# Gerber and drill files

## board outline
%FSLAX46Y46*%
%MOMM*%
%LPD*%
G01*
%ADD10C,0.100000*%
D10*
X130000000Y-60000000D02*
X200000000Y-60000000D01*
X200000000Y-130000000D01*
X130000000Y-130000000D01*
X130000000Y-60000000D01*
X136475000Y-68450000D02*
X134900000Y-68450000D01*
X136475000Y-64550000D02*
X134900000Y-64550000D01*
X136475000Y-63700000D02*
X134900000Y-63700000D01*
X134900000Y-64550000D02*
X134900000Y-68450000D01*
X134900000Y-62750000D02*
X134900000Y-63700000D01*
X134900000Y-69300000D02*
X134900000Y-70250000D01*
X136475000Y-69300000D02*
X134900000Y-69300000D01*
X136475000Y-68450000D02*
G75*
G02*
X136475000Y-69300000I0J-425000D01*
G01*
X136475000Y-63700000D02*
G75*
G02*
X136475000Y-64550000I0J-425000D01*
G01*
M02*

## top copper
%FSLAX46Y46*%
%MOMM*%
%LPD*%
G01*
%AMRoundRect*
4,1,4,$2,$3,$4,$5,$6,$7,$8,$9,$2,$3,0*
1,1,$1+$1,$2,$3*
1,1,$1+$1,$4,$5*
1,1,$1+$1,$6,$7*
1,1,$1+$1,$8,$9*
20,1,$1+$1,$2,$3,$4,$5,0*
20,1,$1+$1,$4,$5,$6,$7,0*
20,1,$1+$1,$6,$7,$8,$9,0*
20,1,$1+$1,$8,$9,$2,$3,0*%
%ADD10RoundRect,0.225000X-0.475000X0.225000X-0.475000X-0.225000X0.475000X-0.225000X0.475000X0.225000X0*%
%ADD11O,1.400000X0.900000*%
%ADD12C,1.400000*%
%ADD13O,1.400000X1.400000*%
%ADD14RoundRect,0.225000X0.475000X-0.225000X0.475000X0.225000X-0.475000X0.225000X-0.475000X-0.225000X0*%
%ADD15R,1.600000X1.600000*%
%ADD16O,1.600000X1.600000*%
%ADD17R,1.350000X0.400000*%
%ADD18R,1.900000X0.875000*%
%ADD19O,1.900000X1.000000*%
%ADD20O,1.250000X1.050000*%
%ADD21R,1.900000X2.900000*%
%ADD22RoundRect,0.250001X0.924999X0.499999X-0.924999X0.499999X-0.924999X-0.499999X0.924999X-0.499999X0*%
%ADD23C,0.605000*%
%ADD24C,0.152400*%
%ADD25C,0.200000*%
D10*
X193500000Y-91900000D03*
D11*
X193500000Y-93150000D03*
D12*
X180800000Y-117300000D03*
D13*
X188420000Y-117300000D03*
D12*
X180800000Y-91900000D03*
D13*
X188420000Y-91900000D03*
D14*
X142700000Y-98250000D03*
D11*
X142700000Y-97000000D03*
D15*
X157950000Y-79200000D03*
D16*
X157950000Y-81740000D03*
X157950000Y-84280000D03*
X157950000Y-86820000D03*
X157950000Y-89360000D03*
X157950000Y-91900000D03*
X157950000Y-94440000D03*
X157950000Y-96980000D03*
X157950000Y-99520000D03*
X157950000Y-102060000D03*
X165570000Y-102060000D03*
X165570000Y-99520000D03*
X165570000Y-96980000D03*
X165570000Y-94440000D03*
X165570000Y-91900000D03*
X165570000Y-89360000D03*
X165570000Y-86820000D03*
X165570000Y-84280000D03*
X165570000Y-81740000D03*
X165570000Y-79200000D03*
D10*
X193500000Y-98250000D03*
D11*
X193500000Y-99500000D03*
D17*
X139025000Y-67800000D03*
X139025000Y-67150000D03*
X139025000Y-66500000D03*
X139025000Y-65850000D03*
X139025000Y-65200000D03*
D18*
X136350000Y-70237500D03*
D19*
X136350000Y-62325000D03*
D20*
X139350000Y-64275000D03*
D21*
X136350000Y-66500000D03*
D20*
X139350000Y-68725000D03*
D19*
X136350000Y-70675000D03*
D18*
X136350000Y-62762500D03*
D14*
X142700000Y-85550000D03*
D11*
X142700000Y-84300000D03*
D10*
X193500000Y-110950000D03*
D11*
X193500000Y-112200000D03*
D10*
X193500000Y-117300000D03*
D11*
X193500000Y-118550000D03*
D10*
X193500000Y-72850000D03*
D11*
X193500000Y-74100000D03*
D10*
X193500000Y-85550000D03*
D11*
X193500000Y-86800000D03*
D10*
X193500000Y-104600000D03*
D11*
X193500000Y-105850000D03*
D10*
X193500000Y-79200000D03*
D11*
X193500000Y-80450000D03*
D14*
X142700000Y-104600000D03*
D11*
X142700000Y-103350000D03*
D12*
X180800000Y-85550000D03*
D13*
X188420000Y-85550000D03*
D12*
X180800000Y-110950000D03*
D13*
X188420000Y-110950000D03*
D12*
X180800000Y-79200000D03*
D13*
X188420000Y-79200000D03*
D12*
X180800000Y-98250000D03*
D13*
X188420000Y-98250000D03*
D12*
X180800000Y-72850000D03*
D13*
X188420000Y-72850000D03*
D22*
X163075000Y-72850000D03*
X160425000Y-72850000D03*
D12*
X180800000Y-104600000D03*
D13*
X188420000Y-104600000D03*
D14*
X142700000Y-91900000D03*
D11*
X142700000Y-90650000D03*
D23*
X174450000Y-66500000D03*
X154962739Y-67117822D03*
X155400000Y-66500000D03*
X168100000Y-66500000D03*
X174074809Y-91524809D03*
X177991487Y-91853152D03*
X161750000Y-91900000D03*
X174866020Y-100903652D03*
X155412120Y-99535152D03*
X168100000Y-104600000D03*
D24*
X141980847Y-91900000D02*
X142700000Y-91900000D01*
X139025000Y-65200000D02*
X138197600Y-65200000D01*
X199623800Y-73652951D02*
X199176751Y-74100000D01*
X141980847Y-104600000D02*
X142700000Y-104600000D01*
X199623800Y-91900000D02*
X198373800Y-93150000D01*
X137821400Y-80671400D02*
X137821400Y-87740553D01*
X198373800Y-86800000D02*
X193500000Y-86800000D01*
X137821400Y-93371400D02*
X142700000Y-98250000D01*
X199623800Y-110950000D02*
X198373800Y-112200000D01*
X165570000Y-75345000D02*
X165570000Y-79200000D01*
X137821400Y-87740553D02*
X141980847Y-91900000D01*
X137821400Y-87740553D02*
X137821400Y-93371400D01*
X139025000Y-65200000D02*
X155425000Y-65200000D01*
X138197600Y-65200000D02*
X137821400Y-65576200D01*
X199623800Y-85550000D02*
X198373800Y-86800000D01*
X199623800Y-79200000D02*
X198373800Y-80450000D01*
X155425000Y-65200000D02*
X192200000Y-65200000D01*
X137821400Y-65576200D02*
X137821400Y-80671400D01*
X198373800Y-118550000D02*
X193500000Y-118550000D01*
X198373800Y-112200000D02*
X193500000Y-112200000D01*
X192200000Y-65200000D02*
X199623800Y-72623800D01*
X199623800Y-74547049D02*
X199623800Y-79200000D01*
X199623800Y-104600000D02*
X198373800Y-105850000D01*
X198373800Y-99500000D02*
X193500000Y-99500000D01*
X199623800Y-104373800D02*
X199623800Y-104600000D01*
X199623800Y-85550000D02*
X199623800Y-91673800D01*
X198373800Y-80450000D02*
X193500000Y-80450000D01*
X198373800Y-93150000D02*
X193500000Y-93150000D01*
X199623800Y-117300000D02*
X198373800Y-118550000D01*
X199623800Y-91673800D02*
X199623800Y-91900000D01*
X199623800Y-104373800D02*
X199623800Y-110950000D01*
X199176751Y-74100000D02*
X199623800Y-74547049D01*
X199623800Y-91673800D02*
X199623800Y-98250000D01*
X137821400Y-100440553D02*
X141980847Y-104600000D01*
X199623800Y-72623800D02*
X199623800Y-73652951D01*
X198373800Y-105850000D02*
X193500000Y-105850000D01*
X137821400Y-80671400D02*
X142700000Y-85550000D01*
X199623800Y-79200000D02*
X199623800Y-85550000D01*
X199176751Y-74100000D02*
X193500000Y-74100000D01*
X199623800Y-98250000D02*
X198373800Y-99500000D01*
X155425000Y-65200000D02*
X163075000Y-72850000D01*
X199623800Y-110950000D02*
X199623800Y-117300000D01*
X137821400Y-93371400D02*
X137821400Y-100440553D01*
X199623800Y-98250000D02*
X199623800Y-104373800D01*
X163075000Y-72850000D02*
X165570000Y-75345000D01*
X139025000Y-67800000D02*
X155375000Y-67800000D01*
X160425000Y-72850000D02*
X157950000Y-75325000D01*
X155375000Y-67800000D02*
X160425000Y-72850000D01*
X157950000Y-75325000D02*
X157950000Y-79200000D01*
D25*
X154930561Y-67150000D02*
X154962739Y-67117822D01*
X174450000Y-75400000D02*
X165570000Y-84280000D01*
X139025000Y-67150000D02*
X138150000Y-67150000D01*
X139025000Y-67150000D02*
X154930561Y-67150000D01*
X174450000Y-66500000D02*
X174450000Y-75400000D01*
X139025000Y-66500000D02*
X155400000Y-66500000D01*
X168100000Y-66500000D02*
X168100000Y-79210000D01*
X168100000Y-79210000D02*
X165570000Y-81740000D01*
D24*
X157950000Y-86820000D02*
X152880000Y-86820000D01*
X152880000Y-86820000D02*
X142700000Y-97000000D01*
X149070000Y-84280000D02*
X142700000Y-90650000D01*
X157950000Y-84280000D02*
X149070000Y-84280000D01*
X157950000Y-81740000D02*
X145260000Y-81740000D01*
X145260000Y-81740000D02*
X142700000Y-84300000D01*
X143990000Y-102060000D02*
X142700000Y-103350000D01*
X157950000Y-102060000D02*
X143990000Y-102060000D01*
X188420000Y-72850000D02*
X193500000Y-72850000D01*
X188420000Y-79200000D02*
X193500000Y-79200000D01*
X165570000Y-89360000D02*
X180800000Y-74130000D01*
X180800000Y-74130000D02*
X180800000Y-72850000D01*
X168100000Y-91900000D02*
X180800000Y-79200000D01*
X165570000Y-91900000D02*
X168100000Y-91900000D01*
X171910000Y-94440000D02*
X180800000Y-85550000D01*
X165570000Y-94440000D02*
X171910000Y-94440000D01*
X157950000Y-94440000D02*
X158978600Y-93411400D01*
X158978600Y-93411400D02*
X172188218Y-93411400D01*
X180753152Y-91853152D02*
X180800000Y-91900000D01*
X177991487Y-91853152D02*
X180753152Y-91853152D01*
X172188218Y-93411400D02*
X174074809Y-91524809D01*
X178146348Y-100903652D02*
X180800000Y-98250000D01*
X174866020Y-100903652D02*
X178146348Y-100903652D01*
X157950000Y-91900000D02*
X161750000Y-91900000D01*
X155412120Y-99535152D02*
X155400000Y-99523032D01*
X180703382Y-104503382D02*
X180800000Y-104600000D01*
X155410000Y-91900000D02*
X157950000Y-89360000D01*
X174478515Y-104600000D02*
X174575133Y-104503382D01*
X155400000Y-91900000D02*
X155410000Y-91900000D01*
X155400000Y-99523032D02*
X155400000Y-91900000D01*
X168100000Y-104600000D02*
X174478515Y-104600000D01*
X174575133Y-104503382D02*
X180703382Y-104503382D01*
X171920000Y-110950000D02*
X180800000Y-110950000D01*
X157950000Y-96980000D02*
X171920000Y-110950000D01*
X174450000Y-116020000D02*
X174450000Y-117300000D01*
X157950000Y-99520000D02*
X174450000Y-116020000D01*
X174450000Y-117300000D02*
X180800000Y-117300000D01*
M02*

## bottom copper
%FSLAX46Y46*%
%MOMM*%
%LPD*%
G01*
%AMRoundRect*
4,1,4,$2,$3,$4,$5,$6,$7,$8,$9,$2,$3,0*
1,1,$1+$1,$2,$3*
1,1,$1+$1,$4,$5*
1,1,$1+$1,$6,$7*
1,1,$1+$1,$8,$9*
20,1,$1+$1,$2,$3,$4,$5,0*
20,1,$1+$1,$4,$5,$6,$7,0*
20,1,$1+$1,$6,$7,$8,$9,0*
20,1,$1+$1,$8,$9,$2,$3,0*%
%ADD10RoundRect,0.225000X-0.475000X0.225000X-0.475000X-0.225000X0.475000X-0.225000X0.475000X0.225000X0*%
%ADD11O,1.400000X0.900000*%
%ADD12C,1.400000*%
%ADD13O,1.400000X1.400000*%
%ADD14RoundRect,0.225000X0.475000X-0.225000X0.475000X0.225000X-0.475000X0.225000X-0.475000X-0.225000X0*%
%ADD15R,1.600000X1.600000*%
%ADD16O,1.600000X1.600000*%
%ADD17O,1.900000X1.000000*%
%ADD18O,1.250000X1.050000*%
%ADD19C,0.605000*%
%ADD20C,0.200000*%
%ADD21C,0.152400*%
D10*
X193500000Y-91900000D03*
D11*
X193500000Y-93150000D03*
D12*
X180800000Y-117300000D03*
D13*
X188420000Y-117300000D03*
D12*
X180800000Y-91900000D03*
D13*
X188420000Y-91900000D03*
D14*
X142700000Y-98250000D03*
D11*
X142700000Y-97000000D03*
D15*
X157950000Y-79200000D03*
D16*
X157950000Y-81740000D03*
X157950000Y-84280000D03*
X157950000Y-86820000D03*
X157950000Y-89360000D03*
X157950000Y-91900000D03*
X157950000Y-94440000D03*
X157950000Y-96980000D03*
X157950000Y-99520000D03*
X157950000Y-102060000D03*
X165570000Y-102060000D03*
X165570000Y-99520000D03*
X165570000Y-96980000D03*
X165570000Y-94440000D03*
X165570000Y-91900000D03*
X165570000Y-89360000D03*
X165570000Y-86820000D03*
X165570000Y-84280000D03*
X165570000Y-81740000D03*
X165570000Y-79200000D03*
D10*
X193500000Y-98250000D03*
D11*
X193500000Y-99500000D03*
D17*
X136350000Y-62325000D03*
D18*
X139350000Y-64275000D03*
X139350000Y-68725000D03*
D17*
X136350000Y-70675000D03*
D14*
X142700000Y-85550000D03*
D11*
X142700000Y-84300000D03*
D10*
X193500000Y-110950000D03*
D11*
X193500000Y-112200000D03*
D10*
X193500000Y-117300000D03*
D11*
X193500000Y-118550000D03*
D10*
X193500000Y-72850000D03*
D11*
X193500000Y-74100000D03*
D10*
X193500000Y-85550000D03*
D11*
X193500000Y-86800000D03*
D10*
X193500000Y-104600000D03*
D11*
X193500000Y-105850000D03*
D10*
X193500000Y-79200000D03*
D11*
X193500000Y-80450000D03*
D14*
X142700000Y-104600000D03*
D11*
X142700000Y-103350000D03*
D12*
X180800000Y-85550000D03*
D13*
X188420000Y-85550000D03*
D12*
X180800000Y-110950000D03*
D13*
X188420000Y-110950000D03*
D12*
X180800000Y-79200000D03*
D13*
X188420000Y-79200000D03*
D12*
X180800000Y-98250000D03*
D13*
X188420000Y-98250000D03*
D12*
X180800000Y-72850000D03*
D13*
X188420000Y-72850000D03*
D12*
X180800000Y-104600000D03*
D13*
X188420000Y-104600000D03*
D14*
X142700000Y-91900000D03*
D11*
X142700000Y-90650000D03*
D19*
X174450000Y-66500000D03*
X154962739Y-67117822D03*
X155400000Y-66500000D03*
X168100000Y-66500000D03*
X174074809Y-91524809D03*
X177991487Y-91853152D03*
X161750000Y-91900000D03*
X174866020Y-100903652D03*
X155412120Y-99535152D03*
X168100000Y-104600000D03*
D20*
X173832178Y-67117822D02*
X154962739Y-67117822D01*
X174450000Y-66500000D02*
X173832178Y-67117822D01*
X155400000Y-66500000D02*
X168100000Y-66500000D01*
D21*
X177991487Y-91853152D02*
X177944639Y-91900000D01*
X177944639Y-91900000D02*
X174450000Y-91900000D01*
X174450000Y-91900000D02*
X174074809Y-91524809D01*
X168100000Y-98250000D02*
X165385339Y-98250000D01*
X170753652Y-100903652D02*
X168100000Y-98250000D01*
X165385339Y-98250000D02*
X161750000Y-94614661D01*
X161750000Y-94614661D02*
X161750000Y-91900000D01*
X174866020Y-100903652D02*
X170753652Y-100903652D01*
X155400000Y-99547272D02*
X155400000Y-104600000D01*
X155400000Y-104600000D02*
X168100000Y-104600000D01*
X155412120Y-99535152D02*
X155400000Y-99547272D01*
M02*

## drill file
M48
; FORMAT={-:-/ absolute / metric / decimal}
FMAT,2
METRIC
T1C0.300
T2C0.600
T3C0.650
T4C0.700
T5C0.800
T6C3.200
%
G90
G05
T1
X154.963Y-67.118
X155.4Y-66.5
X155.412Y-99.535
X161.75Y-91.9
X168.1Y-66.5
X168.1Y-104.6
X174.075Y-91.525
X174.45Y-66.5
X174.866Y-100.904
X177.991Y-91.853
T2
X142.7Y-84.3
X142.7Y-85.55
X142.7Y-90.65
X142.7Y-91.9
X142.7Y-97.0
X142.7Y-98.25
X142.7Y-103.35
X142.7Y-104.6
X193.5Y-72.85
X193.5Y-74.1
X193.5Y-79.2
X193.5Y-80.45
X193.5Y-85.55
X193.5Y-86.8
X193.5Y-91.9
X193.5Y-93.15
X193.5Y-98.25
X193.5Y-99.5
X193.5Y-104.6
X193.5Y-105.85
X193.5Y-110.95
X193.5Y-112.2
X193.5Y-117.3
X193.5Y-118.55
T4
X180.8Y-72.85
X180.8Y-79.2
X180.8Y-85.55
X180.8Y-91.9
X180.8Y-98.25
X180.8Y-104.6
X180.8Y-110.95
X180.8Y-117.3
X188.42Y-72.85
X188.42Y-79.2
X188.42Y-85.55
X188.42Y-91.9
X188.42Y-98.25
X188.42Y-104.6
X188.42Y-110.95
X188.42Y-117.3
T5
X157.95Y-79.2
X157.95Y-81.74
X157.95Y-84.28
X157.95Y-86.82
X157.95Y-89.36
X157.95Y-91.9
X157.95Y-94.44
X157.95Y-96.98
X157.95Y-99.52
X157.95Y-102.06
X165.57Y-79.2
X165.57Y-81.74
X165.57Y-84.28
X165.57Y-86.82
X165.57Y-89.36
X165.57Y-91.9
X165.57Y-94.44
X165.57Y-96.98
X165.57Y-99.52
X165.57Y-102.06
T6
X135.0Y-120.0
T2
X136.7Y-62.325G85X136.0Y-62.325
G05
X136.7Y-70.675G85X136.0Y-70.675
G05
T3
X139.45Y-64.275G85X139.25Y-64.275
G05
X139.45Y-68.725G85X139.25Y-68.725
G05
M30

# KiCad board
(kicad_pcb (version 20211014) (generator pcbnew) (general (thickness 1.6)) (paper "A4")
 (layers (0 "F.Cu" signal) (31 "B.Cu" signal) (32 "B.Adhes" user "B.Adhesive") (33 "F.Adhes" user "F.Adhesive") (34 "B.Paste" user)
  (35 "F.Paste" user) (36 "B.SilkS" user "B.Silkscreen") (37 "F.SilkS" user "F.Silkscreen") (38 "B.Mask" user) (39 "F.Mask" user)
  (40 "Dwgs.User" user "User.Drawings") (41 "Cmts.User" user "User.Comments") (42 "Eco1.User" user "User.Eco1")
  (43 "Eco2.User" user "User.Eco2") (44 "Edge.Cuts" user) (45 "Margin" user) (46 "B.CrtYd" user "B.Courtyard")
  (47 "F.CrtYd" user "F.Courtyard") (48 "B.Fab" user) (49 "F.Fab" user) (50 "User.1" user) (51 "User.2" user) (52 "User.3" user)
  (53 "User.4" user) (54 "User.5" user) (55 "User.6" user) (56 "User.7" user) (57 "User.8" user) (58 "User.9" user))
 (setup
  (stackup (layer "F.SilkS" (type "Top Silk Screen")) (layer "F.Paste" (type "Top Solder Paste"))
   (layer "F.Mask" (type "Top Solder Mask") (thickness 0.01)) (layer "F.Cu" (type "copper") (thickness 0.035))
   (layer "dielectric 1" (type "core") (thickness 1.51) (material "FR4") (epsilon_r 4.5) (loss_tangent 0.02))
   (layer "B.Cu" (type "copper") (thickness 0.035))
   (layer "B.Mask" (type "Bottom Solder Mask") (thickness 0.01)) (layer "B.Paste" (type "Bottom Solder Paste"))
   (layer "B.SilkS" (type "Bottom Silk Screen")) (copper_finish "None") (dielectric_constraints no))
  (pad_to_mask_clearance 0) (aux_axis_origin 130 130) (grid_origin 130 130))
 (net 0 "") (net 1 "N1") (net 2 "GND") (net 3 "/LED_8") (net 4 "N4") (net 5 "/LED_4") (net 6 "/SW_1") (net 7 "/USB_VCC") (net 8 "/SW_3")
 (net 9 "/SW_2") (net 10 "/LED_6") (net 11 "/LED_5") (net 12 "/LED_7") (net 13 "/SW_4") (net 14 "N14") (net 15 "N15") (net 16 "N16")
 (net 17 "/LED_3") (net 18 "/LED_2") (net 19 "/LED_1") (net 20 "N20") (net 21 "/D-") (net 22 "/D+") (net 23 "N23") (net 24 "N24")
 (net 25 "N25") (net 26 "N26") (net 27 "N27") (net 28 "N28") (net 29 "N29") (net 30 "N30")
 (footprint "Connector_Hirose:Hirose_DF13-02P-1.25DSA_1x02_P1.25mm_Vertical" (layer "F.Cu") (at 193.5 91.9 -90)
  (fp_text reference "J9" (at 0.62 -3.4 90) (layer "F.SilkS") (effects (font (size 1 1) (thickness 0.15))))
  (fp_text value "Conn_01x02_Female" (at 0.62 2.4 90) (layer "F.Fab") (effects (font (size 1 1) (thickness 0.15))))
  (pad "1" thru_hole roundrect (at 0 0 270) (size 0.9 1.4) (drill 0.6) (layers *.Cu *.Mask) (roundrect_rratio 0.25) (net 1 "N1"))
  (pad "2" thru_hole oval (at 1.25 0 270) (size 0.9 1.4) (drill 0.6) (layers *.Cu *.Mask) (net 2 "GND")))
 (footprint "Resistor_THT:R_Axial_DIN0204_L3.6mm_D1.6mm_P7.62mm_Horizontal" (layer "F.Cu") (at 180.8 117.3)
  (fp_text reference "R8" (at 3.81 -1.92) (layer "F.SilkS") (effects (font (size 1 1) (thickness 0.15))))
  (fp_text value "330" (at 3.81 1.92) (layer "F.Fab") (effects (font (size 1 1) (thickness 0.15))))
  (pad "1" thru_hole circle (at 0 0) (size 1.4 1.4) (drill 0.7) (layers *.Cu *.Mask) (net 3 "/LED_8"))
  (pad "2" thru_hole oval (at 7.62 0) (size 1.4 1.4) (drill 0.7) (layers *.Cu *.Mask) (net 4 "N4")))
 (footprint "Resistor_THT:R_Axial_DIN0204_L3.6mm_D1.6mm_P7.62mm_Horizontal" (layer "F.Cu") (at 180.8 91.9)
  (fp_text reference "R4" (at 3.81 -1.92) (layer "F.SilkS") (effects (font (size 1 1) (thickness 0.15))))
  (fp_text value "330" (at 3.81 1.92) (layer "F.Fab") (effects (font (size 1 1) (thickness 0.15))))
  (pad "1" thru_hole circle (at 0 0) (size 1.4 1.4) (drill 0.7) (layers *.Cu *.Mask) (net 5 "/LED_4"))
  (pad "2" thru_hole oval (at 7.62 0) (size 1.4 1.4) (drill 0.7) (layers *.Cu *.Mask) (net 1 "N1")))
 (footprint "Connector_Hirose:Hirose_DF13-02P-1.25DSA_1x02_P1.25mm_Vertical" (layer "F.Cu") (at 142.7 98.25 90)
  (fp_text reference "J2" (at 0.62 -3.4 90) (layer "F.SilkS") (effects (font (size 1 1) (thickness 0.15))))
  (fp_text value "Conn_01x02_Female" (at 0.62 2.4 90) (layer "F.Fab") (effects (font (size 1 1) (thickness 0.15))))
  (pad "1" thru_hole roundrect (at 0 0 90) (size 0.9 1.4) (drill 0.6) (layers *.Cu *.Mask) (roundrect_rratio 0.25) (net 2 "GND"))
  (pad "2" thru_hole oval (at 1.25 0 90) (size 0.9 1.4) (drill 0.6) (layers *.Cu *.Mask) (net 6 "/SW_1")))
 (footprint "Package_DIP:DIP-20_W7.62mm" (layer "F.Cu") (at 157.95 79.2)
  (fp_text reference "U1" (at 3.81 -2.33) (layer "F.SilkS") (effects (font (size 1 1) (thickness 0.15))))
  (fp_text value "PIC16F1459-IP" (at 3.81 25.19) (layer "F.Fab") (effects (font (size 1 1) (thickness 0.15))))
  (pad "1" thru_hole rect (at 0 0) (size 1.6 1.6) (drill 0.8) (layers *.Cu *.Mask) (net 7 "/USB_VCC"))
  (pad "2" thru_hole oval (at 0 2.54) (size 1.6 1.6) (drill 0.8) (layers *.Cu *.Mask) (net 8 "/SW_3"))
  (pad "3" thru_hole oval (at 0 5.08) (size 1.6 1.6) (drill 0.8) (layers *.Cu *.Mask) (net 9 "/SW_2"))
  (pad "4" thru_hole oval (at 0 7.62) (size 1.6 1.6) (drill 0.8) (layers *.Cu *.Mask) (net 6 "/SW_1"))
  (pad "5" thru_hole oval (at 0 10.16) (size 1.6 1.6) (drill 0.8) (layers *.Cu *.Mask) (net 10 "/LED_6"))
  (pad "6" thru_hole oval (at 0 12.7) (size 1.6 1.6) (drill 0.8) (layers *.Cu *.Mask) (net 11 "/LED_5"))
  (pad "7" thru_hole oval (at 0 15.24) (size 1.6 1.6) (drill 0.8) (layers *.Cu *.Mask) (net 5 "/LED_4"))
  (pad "8" thru_hole oval (at 0 17.78) (size 1.6 1.6) (drill 0.8) (layers *.Cu *.Mask) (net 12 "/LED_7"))
  (pad "9" thru_hole oval (at 0 20.32) (size 1.6 1.6) (drill 0.8) (layers *.Cu *.Mask) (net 3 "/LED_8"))
  (pad "10" thru_hole oval (at 0 22.86) (size 1.6 1.6) (drill 0.8) (layers *.Cu *.Mask) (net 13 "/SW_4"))
  (pad "11" thru_hole oval (at 7.62 22.86) (size 1.6 1.6) (drill 0.8) (layers *.Cu *.Mask) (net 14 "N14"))
  (pad "12" thru_hole oval (at 7.62 20.32) (size 1.6 1.6) (drill 0.8) (layers *.Cu *.Mask) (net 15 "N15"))
  (pad "13" thru_hole oval (at 7.62 17.78) (size 1.6 1.6) (drill 0.8) (layers *.Cu *.Mask) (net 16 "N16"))
  (pad "14" thru_hole oval (at 7.62 15.24) (size 1.6 1.6) (drill 0.8) (layers *.Cu *.Mask) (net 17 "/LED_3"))
  (pad "15" thru_hole oval (at 7.62 12.7) (size 1.6 1.6) (drill 0.8) (layers *.Cu *.Mask) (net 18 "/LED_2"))
  (pad "16" thru_hole oval (at 7.62 10.16) (size 1.6 1.6) (drill 0.8) (layers *.Cu *.Mask) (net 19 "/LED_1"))
  (pad "17" thru_hole oval (at 7.62 7.62) (size 1.6 1.6) (drill 0.8) (layers *.Cu *.Mask) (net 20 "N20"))
  (pad "18" thru_hole oval (at 7.62 5.08) (size 1.6 1.6) (drill 0.8) (layers *.Cu *.Mask) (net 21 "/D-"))
  (pad "19" thru_hole oval (at 7.62 2.54) (size 1.6 1.6) (drill 0.8) (layers *.Cu *.Mask) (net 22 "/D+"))
  (pad "20" thru_hole oval (at 7.62 0) (size 1.6 1.6) (drill 0.8) (layers *.Cu *.Mask) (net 2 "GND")))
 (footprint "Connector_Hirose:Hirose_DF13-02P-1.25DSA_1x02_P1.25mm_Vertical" (layer "F.Cu") (at 193.5 98.25 -90)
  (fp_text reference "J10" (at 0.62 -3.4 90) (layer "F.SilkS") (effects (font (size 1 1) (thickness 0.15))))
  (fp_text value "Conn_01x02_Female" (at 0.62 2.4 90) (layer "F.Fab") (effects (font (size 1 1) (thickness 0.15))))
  (pad "1" thru_hole roundrect (at 0 0 270) (size 0.9 1.4) (drill 0.6) (layers *.Cu *.Mask) (roundrect_rratio 0.25) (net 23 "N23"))
  (pad "2" thru_hole oval (at 1.25 0 270) (size 0.9 1.4) (drill 0.6) (layers *.Cu *.Mask) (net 2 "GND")))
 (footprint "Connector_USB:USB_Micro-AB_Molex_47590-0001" (layer "F.Cu") (at 136.35 66.5 -90)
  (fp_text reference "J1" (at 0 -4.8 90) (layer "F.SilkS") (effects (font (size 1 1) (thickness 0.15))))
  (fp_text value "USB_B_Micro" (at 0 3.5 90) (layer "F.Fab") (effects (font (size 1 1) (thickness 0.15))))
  (fp_line (start 1.95 -0.125) (end 1.95 1.45) (layer "Edge.Cuts") (width 0.1))
  (fp_line (start -1.95 -0.125) (end -1.95 1.45) (layer "Edge.Cuts") (width 0.1))
  (fp_line (start -2.8 -0.125) (end -2.8 1.45) (layer "Edge.Cuts") (width 0.1))
  (fp_line (start -1.95 1.45) (end 1.95 1.45) (layer "Edge.Cuts") (width 0.1))
  (fp_line (start -3.75 1.45) (end -2.8 1.45) (layer "Edge.Cuts") (width 0.1))
  (fp_line (start 2.8 1.45) (end 3.75 1.45) (layer "Edge.Cuts") (width 0.1))
  (fp_line (start 2.8 -0.125) (end 2.8 1.45) (layer "Edge.Cuts") (width 0.1))
  (fp_arc (start 1.95 -0.125) (mid 2.375 -0.55) (end 2.8 -0.125) (layer "Edge.Cuts") (width 0.1))
  (fp_arc (start -2.8 -0.125) (mid -2.375 -0.55) (end -1.95 -0.125) (layer "Edge.Cuts") (width 0.1))
  (pad "" smd rect (at -3.5 0 270) (size 0.3 0.85) (layers "F.Paste"))
  (pad "" smd rect (at 3.5 0 270) (size 0.3 0.85) (layers "F.Paste"))
  (pad "1" smd rect (at 1.3 -2.675 270) (size 0.4 1.35) (layers "F.Cu" "F.Paste" "F.Mask") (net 7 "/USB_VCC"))
  (pad "2" smd rect (at 0.65 -2.675 270) (size 0.4 1.35) (layers "F.Cu" "F.Paste" "F.Mask") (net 21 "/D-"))
  (pad "3" smd rect (at 0 -2.675 270) (size 0.4 1.35) (layers "F.Cu" "F.Paste" "F.Mask") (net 22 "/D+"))
  (pad "4" smd rect (at -0.65 -2.675 270) (size 0.4 1.35) (layers "F.Cu" "F.Paste" "F.Mask") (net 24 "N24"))
  (pad "5" smd rect (at -1.3 -2.675 270) (size 0.4 1.35) (layers "F.Cu" "F.Paste" "F.Mask") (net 2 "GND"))
  (pad "6" smd rect (at 3.7375 0 270) (size 0.875 1.9) (layers "F.Cu" "F.Mask") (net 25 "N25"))
  (pad "6" thru_hole oval (at -4.175 0 270) (size 1 1.9) (drill oval 0.6 1.3) (layers *.Cu *.Mask) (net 25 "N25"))
  (pad "6" thru_hole oval (at -2.225 -3 270) (size 1.05 1.25) (drill oval 0.65 0.85) (layers *.Cu *.Mask) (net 25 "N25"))
  (pad "6" smd rect (at 0 0 270) (size 2.9 1.9) (layers "F.Cu" "F.Paste" "F.Mask") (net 25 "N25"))
  (pad "6" thru_hole oval (at 2.225 -3 270) (size 1.05 1.25) (drill oval 0.65 0.85) (layers *.Cu *.Mask) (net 25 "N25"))
  (pad "6" thru_hole oval (at 4.175 0 270) (size 1 1.9) (drill oval 0.6 1.3) (layers *.Cu *.Mask) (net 25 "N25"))
  (pad "6" smd rect (at -3.7375 0 270) (size 0.875 1.9) (layers "F.Cu" "F.Mask") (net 25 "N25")))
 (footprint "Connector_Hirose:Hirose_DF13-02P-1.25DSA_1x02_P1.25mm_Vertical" (layer "F.Cu") (at 142.7 85.55 90)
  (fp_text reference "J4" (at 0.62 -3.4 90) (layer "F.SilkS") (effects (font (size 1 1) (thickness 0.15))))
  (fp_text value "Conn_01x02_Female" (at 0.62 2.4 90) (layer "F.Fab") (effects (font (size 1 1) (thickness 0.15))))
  (pad "1" thru_hole roundrect (at 0 0 90) (size 0.9 1.4) (drill 0.6) (layers *.Cu *.Mask) (roundrect_rratio 0.25) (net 2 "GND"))
  (pad "2" thru_hole oval (at 1.25 0 90) (size 0.9 1.4) (drill 0.6) (layers *.Cu *.Mask) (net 8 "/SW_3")))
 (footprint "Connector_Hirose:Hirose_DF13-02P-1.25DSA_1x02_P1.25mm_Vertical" (layer "F.Cu") (at 193.5 110.95 -90)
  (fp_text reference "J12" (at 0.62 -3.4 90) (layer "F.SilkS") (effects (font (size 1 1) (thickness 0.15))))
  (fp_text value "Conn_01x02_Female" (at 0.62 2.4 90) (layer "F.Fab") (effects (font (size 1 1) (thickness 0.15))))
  (pad "1" thru_hole roundrect (at 0 0 270) (size 0.9 1.4) (drill 0.6) (layers *.Cu *.Mask) (roundrect_rratio 0.25) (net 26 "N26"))
  (pad "2" thru_hole oval (at 1.25 0 270) (size 0.9 1.4) (drill 0.6) (layers *.Cu *.Mask) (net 2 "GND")))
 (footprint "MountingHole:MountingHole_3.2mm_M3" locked (layer "F.Cu") (at 135 120)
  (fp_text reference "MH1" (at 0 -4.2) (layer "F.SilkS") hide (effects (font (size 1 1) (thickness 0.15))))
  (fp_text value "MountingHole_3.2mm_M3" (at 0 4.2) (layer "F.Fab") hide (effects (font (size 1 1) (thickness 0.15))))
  (pad "" np_thru_hole circle locked (at 0 0) (size 3.2 3.2) (drill 3.2) (layers *.Cu *.Mask)))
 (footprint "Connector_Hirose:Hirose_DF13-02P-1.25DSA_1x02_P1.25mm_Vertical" (layer "F.Cu") (at 193.5 117.3 -90)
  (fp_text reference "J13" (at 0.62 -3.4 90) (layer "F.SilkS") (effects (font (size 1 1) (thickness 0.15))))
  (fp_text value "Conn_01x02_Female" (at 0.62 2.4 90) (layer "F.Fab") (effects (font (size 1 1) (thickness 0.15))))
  (pad "1" thru_hole roundrect (at 0 0 270) (size 0.9 1.4) (drill 0.6) (layers *.Cu *.Mask) (roundrect_rratio 0.25) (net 4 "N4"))
  (pad "2" thru_hole oval (at 1.25 0 270) (size 0.9 1.4) (drill 0.6) (layers *.Cu *.Mask) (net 2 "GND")))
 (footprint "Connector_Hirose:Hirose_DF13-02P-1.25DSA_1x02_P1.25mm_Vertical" (layer "F.Cu") (at 193.5 72.85 -90)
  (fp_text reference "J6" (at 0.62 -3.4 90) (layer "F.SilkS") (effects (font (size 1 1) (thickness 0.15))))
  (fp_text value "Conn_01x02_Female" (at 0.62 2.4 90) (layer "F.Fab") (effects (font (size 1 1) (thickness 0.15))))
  (pad "1" thru_hole roundrect (at 0 0 270) (size 0.9 1.4) (drill 0.6) (layers *.Cu *.Mask) (roundrect_rratio 0.25) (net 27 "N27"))
  (pad "2" thru_hole oval (at 1.25 0 270) (size 0.9 1.4) (drill 0.6) (layers *.Cu *.Mask) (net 2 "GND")))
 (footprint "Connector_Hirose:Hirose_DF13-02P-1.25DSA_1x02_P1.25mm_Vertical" (layer "F.Cu") (at 193.5 85.55 -90)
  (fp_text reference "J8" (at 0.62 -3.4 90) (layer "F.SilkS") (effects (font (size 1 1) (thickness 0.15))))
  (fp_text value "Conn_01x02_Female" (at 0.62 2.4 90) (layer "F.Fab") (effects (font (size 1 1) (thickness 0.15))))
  (pad "1" thru_hole roundrect (at 0 0 270) (size 0.9 1.4) (drill 0.6) (layers *.Cu *.Mask) (roundrect_rratio 0.25) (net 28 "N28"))
  (pad "2" thru_hole oval (at 1.25 0 270) (size 0.9 1.4) (drill 0.6) (layers *.Cu *.Mask) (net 2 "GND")))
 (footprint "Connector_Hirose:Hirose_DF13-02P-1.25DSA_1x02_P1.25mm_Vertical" (layer "F.Cu") (at 193.5 104.6 -90)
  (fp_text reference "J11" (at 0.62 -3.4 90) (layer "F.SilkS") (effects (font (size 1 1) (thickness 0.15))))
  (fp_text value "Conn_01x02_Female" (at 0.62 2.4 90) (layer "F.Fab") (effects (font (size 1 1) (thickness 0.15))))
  (pad "1" thru_hole roundrect (at 0 0 270) (size 0.9 1.4) (drill 0.6) (layers *.Cu *.Mask) (roundrect_rratio 0.25) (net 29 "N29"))
  (pad "2" thru_hole oval (at 1.25 0 270) (size 0.9 1.4) (drill 0.6) (layers *.Cu *.Mask) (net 2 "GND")))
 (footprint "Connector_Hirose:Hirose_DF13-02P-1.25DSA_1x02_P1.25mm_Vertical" (layer "F.Cu") (at 193.5 79.2 -90)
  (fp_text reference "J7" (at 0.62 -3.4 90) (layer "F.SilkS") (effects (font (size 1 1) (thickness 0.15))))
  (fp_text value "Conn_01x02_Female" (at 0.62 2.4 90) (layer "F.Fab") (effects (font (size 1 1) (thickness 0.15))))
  (pad "1" thru_hole roundrect (at 0 0 270) (size 0.9 1.4) (drill 0.6) (layers *.Cu *.Mask) (roundrect_rratio 0.25) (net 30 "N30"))
  (pad "2" thru_hole oval (at 1.25 0 270) (size 0.9 1.4) (drill 0.6) (layers *.Cu *.Mask) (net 2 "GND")))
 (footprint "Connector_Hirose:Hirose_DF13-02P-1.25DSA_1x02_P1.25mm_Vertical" (layer "F.Cu") (at 142.7 104.6 90)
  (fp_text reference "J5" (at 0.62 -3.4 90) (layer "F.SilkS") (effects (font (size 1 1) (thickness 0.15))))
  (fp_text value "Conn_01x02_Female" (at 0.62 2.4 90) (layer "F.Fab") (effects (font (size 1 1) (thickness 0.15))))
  (pad "1" thru_hole roundrect (at 0 0 90) (size 0.9 1.4) (drill 0.6) (layers *.Cu *.Mask) (roundrect_rratio 0.25) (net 2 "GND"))
  (pad "2" thru_hole oval (at 1.25 0 90) (size 0.9 1.4) (drill 0.6) (layers *.Cu *.Mask) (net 13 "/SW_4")))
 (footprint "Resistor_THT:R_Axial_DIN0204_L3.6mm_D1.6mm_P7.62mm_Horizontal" (layer "F.Cu") (at 180.8 85.55)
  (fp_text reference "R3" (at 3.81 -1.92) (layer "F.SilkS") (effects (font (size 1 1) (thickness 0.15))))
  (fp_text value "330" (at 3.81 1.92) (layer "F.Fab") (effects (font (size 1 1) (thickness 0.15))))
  (pad "1" thru_hole circle (at 0 0) (size 1.4 1.4) (drill 0.7) (layers *.Cu *.Mask) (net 17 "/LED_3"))
  (pad "2" thru_hole oval (at 7.62 0) (size 1.4 1.4) (drill 0.7) (layers *.Cu *.Mask) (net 28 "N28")))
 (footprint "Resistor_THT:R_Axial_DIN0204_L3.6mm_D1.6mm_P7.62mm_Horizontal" (layer "F.Cu") (at 180.8 110.95)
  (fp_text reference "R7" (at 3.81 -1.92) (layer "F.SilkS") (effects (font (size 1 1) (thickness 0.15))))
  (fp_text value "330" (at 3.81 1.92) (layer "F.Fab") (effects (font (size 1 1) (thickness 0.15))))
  (pad "1" thru_hole circle (at 0 0) (size 1.4 1.4) (drill 0.7) (layers *.Cu *.Mask) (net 12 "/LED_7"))
  (pad "2" thru_hole oval (at 7.62 0) (size 1.4 1.4) (drill 0.7) (layers *.Cu *.Mask) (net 26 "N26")))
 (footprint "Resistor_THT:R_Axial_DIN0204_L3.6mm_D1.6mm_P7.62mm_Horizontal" (layer "F.Cu") (at 180.8 79.2)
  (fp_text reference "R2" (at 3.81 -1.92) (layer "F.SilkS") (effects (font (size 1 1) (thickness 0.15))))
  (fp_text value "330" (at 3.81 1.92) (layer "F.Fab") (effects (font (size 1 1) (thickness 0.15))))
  (pad "1" thru_hole circle (at 0 0) (size 1.4 1.4) (drill 0.7) (layers *.Cu *.Mask) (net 18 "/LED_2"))
  (pad "2" thru_hole oval (at 7.62 0) (size 1.4 1.4) (drill 0.7) (layers *.Cu *.Mask) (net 30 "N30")))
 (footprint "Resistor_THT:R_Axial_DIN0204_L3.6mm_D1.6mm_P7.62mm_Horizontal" (layer "F.Cu") (at 180.8 98.25)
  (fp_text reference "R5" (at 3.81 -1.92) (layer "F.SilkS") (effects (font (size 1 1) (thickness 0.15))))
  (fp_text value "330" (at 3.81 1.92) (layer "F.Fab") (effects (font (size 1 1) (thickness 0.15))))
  (pad "1" thru_hole circle (at 0 0) (size 1.4 1.4) (drill 0.7) (layers *.Cu *.Mask) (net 11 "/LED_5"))
  (pad "2" thru_hole oval (at 7.62 0) (size 1.4 1.4) (drill 0.7) (layers *.Cu *.Mask) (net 23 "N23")))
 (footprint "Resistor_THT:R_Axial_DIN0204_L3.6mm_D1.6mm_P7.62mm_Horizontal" (layer "F.Cu") (at 180.8 72.85)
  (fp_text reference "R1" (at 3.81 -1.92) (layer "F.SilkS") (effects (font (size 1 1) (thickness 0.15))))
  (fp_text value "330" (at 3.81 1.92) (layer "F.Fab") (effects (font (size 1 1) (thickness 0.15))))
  (pad "1" thru_hole circle (at 0 0) (size 1.4 1.4) (drill 0.7) (layers *.Cu *.Mask) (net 19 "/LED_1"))
  (pad "2" thru_hole oval (at 7.62 0) (size 1.4 1.4) (drill 0.7) (layers *.Cu *.Mask) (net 27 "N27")))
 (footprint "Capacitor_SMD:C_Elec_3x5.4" (layer "F.Cu") (at 161.75 72.85 180)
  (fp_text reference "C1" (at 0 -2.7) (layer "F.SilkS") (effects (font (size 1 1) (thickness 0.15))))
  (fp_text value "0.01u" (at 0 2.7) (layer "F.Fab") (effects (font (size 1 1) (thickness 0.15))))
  (pad "1" smd roundrect (at -1.325 0 180) (size 2.35 1.5) (layers "F.Cu" "F.Paste" "F.Mask") (roundrect_rratio 0.166667) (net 2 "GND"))
  (pad "2" smd roundrect (at 1.325 0 180) (size 2.35 1.5) (layers "F.Cu" "F.Paste" "F.Mask") (roundrect_rratio 0.166667) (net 7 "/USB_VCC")))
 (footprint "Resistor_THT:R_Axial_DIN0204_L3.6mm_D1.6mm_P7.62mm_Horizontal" (layer "F.Cu") (at 180.8 104.6)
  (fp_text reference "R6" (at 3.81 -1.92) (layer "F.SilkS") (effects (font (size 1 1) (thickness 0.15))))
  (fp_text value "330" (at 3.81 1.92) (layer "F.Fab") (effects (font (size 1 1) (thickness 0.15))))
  (pad "1" thru_hole circle (at 0 0) (size 1.4 1.4) (drill 0.7) (layers *.Cu *.Mask) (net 10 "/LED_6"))
  (pad "2" thru_hole oval (at 7.62 0) (size 1.4 1.4) (drill 0.7) (layers *.Cu *.Mask) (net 29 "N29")))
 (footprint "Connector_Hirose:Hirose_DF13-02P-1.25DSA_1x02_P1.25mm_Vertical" (layer "F.Cu") (at 142.7 91.9 90)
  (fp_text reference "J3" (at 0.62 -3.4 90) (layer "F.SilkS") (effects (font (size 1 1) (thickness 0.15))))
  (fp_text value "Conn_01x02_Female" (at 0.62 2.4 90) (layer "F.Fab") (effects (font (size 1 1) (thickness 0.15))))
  (pad "1" thru_hole roundrect (at 0 0 90) (size 0.9 1.4) (drill 0.6) (layers *.Cu *.Mask) (roundrect_rratio 0.25) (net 2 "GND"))
  (pad "2" thru_hole oval (at 1.25 0 90) (size 0.9 1.4) (drill 0.6) (layers *.Cu *.Mask) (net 9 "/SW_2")))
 (gr_rect locked (start 130 130) (end 200 60) (layer "Edge.Cuts") (width 0.1) (fill none))
 (segment (start 141.980847 91.9) (end 142.7 91.9) (width 0.1524) (layer "F.Cu") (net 2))
 (segment (start 139.025 65.2) (end 138.1976 65.2) (width 0.1524) (layer "F.Cu") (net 2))
 (segment (start 199.6238 73.652951) (end 199.176751 74.1) (width 0.1524) (layer "F.Cu") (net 2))
 (segment (start 141.980847 104.6) (end 142.7 104.6) (width 0.1524) (layer "F.Cu") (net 2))
 (segment (start 199.6238 91.9) (end 198.3738 93.15) (width 0.1524) (layer "F.Cu") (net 2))
 (segment (start 137.8214 80.6714) (end 137.8214 87.740553) (width 0.1524) (layer "F.Cu") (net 2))
 (segment (start 198.3738 86.8) (end 193.5 86.8) (width 0.1524) (layer "F.Cu") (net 2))
 (segment (start 137.8214 93.3714) (end 142.7 98.25) (width 0.1524) (layer "F.Cu") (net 2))
 (segment (start 199.6238 110.95) (end 198.3738 112.2) (width 0.1524) (layer "F.Cu") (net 2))
 (segment (start 165.57 75.345) (end 165.57 79.2) (width 0.1524) (layer "F.Cu") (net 2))
 (segment (start 137.8214 87.740553) (end 141.980847 91.9) (width 0.1524) (layer "F.Cu") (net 2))
 (segment (start 137.8214 87.740553) (end 137.8214 93.3714) (width 0.1524) (layer "F.Cu") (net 2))
 (segment (start 139.025 65.2) (end 155.425 65.2) (width 0.1524) (layer "F.Cu") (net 2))
 (segment (start 138.1976 65.2) (end 137.8214 65.5762) (width 0.1524) (layer "F.Cu") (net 2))
 (segment (start 199.6238 85.55) (end 198.3738 86.8) (width 0.1524) (layer "F.Cu") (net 2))
 (segment (start 199.6238 79.2) (end 198.3738 80.45) (width 0.1524) (layer "F.Cu") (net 2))
 (segment (start 155.425 65.2) (end 192.2 65.2) (width 0.1524) (layer "F.Cu") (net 2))
 (segment (start 137.8214 65.5762) (end 137.8214 80.6714) (width 0.1524) (layer "F.Cu") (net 2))
 (segment (start 198.3738 118.55) (end 193.5 118.55) (width 0.1524) (layer "F.Cu") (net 2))
 (segment (start 198.3738 112.2) (end 193.5 112.2) (width 0.1524) (layer "F.Cu") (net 2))
 (segment (start 192.2 65.2) (end 199.6238 72.6238) (width 0.1524) (layer "F.Cu") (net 2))
 (segment (start 199.6238 74.547049) (end 199.6238 79.2) (width 0.1524) (layer "F.Cu") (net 2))
 (segment (start 199.6238 104.6) (end 198.3738 105.85) (width 0.1524) (layer "F.Cu") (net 2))
 (segment (start 198.3738 99.5) (end 193.5 99.5) (width 0.1524) (layer "F.Cu") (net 2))
 (segment (start 199.6238 104.3738) (end 199.6238 104.6) (width 0.1524) (layer "F.Cu") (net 2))
 (segment (start 199.6238 85.55) (end 199.6238 91.6738) (width 0.1524) (layer "F.Cu") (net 2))
 (segment (start 198.3738 80.45) (end 193.5 80.45) (width 0.1524) (layer "F.Cu") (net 2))
 (segment (start 198.3738 93.15) (end 193.5 93.15) (width 0.1524) (layer "F.Cu") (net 2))
 (segment (start 199.6238 117.3) (end 198.3738 118.55) (width 0.1524) (layer "F.Cu") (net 2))
 (segment (start 199.6238 91.6738) (end 199.6238 91.9) (width 0.1524) (layer "F.Cu") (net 2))
 (segment (start 199.6238 104.3738) (end 199.6238 110.95) (width 0.1524) (layer "F.Cu") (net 2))
 (segment (start 199.176751 74.1) (end 199.6238 74.547049) (width 0.1524) (layer "F.Cu") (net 2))
 (segment (start 199.6238 91.6738) (end 199.6238 98.25) (width 0.1524) (layer "F.Cu") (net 2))
 (segment (start 137.8214 100.440553) (end 141.980847 104.6) (width 0.1524) (layer "F.Cu") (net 2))
 (segment (start 199.6238 72.6238) (end 199.6238 73.652951) (width 0.1524) (layer "F.Cu") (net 2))
 (segment (start 198.3738 105.85) (end 193.5 105.85) (width 0.1524) (layer "F.Cu") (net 2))
 (segment (start 137.8214 80.6714) (end 142.7 85.55) (width 0.1524) (layer "F.Cu") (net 2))
 (segment (start 199.6238 79.2) (end 199.6238 85.55) (width 0.1524) (layer "F.Cu") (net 2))
 (segment (start 199.176751 74.1) (end 193.5 74.1) (width 0.1524) (layer "F.Cu") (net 2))
 (segment (start 199.6238 98.25) (end 198.3738 99.5) (width 0.1524) (layer "F.Cu") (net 2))
 (segment (start 155.425 65.2) (end 163.075 72.85) (width 0.1524) (layer "F.Cu") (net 2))
 (segment (start 199.6238 110.95) (end 199.6238 117.3) (width 0.1524) (layer "F.Cu") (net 2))
 (segment (start 137.8214 93.3714) (end 137.8214 100.440553) (width 0.1524) (layer "F.Cu") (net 2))
 (segment (start 199.6238 98.25) (end 199.6238 104.3738) (width 0.1524) (layer "F.Cu") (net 2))
 (segment (start 163.075 72.85) (end 165.57 75.345) (width 0.1524) (layer "F.Cu") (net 2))
 (segment (start 139.025 67.8) (end 155.375 67.8) (width 0.1524) (layer "F.Cu") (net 7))
 (segment (start 160.425 72.85) (end 157.95 75.325) (width 0.1524) (layer "F.Cu") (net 7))
 (segment (start 155.375 67.8) (end 160.425 72.85) (width 0.1524) (layer "F.Cu") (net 7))
 (segment (start 157.95 75.325) (end 157.95 79.2) (width 0.1524) (layer "F.Cu") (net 7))
 (segment (start 154.930561 67.15) (end 154.962739 67.117822) (width 0.2) (layer "F.Cu") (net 21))
 (segment (start 174.45 75.4) (end 165.57 84.28) (width 0.2) (layer "F.Cu") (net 21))
 (segment (start 139.025 67.15) (end 138.15 67.15) (width 0.2) (layer "F.Cu") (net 21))
 (segment (start 139.025 67.15) (end 154.930561 67.15) (width 0.2) (layer "F.Cu") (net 21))
 (segment (start 174.45 66.5) (end 174.45 75.4) (width 0.2) (layer "F.Cu") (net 21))
 (via (at 174.45 66.5) (size 0.605) (drill 0.3) (layers "F.Cu" "B.Cu") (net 21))
 (via (at 154.962739 67.117822) (size 0.605) (drill 0.3) (layers "F.Cu" "B.Cu") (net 21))
 (segment (start 173.832178 67.117822) (end 154.962739 67.117822) (width 0.2) (layer "B.Cu") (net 21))
 (segment (start 174.45 66.5) (end 173.832178 67.117822) (width 0.2) (layer "B.Cu") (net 21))
 (segment (start 139.025 66.5) (end 155.4 66.5) (width 0.2) (layer "F.Cu") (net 22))
 (segment (start 168.1 66.5) (end 168.1 79.21) (width 0.2) (layer "F.Cu") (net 22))
 (segment (start 168.1 79.21) (end 165.57 81.74) (width 0.2) (layer "F.Cu") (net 22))
 (via (at 155.4 66.5) (size 0.605) (drill 0.3) (layers "F.Cu" "B.Cu") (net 22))
 (via (at 168.1 66.5) (size 0.605) (drill 0.3) (layers "F.Cu" "B.Cu") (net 22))
 (segment (start 155.4 66.5) (end 168.1 66.5) (width 0.2) (layer "B.Cu") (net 22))
 (segment (start 157.95 86.82) (end 152.88 86.82) (width 0.1524) (layer "F.Cu") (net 6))
 (segment (start 152.88 86.82) (end 142.7 97) (width 0.1524) (layer "F.Cu") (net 6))
 (segment (start 149.07 84.28) (end 142.7 90.65) (width 0.1524) (layer "F.Cu") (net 9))
 (segment (start 157.95 84.28) (end 149.07 84.28) (width 0.1524) (layer "F.Cu") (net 9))
 (segment (start 157.95 81.74) (end 145.26 81.74) (width 0.1524) (layer "F.Cu") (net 8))
 (segment (start 145.26 81.74) (end 142.7 84.3) (width 0.1524) (layer "F.Cu") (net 8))
 (segment (start 143.99 102.06) (end 142.7 103.35) (width 0.1524) (layer "F.Cu") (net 13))
 (segment (start 157.95 102.06) (end 143.99 102.06) (width 0.1524) (layer "F.Cu") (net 13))
 (segment (start 188.42 72.85) (end 193.5 72.85) (width 0.1524) (layer "F.Cu") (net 27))
 (segment (start 188.42 79.2) (end 193.5 79.2) (width 0.1524) (layer "F.Cu") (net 30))
 (segment (start 165.57 89.36) (end 180.8 74.13) (width 0.1524) (layer "F.Cu") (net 19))
 (segment (start 180.8 74.13) (end 180.8 72.85) (width 0.1524) (layer "F.Cu") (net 19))
 (segment (start 168.1 91.9) (end 180.8 79.2) (width 0.1524) (layer "F.Cu") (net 18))
 (segment (start 165.57 91.9) (end 168.1 91.9) (width 0.1524) (layer "F.Cu") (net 18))
 (segment (start 171.91 94.44) (end 180.8 85.55) (width 0.1524) (layer "F.Cu") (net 17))
 (segment (start 165.57 94.44) (end 171.91 94.44) (width 0.1524) (layer "F.Cu") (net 17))
 (segment (start 157.95 94.44) (end 158.9786 93.4114) (width 0.1524) (layer "F.Cu") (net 5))
 (segment (start 158.9786 93.4114) (end 172.188218 93.4114) (width 0.1524) (layer "F.Cu") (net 5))
 (segment (start 180.753152 91.853152) (end 180.8 91.9) (width 0.1524) (layer "F.Cu") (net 5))
 (segment (start 177.991487 91.853152) (end 180.753152 91.853152) (width 0.1524) (layer "F.Cu") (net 5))
 (segment (start 172.188218 93.4114) (end 174.074809 91.524809) (width 0.1524) (layer "F.Cu") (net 5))
 (via (at 174.074809 91.524809) (size 0.605) (drill 0.3) (layers "F.Cu" "B.Cu") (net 5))
 (via (at 177.991487 91.853152) (size 0.605) (drill 0.3) (layers "F.Cu" "B.Cu") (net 5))
 (segment (start 177.991487 91.853152) (end 177.944639 91.9) (width 0.1524) (layer "B.Cu") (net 5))
 (segment (start 177.944639 91.9) (end 174.45 91.9) (width 0.1524) (layer "B.Cu") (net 5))
 (segment (start 174.45 91.9) (end 174.074809 91.524809) (width 0.1524) (layer "B.Cu") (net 5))
 (segment (start 178.146348 100.903652) (end 180.8 98.25) (width 0.1524) (layer "F.Cu") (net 11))
 (segment (start 174.86602 100.903652) (end 178.146348 100.903652) (width 0.1524) (layer "F.Cu") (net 11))
 (segment (start 157.95 91.9) (end 161.75 91.9) (width 0.1524) (layer "F.Cu") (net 11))
 (via (at 161.75 91.9) (size 0.605) (drill 0.3) (layers "F.Cu" "B.Cu") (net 11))
 (via (at 174.86602 100.903652) (size 0.605) (drill 0.3) (layers "F.Cu" "B.Cu") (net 11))
 (segment (start 168.1 98.25) (end 165.385339 98.25) (width 0.1524) (layer "B.Cu") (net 11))
 (segment (start 170.753652 100.903652) (end 168.1 98.25) (width 0.1524) (layer "B.Cu") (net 11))
 (segment (start 165.385339 98.25) (end 161.75 94.614661) (width 0.1524) (layer "B.Cu") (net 11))
 (segment (start 161.75 94.614661) (end 161.75 91.9) (width 0.1524) (layer "B.Cu") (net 11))
 (segment (start 174.86602 100.903652) (end 170.753652 100.903652) (width 0.1524) (layer "B.Cu") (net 11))
 (segment (start 155.41212 99.535152) (end 155.4 99.523032) (width 0.1524) (layer "F.Cu") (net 10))
 (segment (start 180.703382 104.503382) (end 180.8 104.6) (width 0.1524) (layer "F.Cu") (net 10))
 (segment (start 155.41 91.9) (end 157.95 89.36) (width 0.1524) (layer "F.Cu") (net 10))
 (segment (start 174.478515 104.6) (end 174.575133 104.503382) (width 0.1524) (layer "F.Cu") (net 10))
 (segment (start 155.4 91.9) (end 155.41 91.9) (width 0.1524) (layer "F.Cu") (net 10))
 (segment (start 155.4 99.523032) (end 155.4 91.9) (width 0.1524) (layer "F.Cu") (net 10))
 (segment (start 168.1 104.6) (end 174.478515 104.6) (width 0.1524) (layer "F.Cu") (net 10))
 (segment (start 174.575133 104.503382) (end 180.703382 104.503382) (width 0.1524) (layer "F.Cu") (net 10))
 (via (at 155.41212 99.535152) (size 0.605) (drill 0.3) (layers "F.Cu" "B.Cu") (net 10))
 (via (at 168.1 104.6) (size 0.605) (drill 0.3) (layers "F.Cu" "B.Cu") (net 10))
 (segment (start 155.4 99.547272) (end 155.4 104.6) (width 0.1524) (layer "B.Cu") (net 10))
 (segment (start 155.4 104.6) (end 168.1 104.6) (width 0.1524) (layer "B.Cu") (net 10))
 (segment (start 155.41212 99.535152) (end 155.4 99.547272) (width 0.1524) (layer "B.Cu") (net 10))
 (segment (start 171.92 110.95) (end 180.8 110.95) (width 0.1524) (layer "F.Cu") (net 12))
 (segment (start 157.95 96.98) (end 171.92 110.95) (width 0.1524) (layer "F.Cu") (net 12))
 (segment (start 174.45 116.02) (end 174.45 117.3) (width 0.1524) (layer "F.Cu") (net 3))
 (segment (start 157.95 99.52) (end 174.45 116.02) (width 0.1524) (layer "F.Cu") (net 3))
 (segment (start 174.45 117.3) (end 180.8 117.3) (width 0.1524) (layer "F.Cu") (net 3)))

